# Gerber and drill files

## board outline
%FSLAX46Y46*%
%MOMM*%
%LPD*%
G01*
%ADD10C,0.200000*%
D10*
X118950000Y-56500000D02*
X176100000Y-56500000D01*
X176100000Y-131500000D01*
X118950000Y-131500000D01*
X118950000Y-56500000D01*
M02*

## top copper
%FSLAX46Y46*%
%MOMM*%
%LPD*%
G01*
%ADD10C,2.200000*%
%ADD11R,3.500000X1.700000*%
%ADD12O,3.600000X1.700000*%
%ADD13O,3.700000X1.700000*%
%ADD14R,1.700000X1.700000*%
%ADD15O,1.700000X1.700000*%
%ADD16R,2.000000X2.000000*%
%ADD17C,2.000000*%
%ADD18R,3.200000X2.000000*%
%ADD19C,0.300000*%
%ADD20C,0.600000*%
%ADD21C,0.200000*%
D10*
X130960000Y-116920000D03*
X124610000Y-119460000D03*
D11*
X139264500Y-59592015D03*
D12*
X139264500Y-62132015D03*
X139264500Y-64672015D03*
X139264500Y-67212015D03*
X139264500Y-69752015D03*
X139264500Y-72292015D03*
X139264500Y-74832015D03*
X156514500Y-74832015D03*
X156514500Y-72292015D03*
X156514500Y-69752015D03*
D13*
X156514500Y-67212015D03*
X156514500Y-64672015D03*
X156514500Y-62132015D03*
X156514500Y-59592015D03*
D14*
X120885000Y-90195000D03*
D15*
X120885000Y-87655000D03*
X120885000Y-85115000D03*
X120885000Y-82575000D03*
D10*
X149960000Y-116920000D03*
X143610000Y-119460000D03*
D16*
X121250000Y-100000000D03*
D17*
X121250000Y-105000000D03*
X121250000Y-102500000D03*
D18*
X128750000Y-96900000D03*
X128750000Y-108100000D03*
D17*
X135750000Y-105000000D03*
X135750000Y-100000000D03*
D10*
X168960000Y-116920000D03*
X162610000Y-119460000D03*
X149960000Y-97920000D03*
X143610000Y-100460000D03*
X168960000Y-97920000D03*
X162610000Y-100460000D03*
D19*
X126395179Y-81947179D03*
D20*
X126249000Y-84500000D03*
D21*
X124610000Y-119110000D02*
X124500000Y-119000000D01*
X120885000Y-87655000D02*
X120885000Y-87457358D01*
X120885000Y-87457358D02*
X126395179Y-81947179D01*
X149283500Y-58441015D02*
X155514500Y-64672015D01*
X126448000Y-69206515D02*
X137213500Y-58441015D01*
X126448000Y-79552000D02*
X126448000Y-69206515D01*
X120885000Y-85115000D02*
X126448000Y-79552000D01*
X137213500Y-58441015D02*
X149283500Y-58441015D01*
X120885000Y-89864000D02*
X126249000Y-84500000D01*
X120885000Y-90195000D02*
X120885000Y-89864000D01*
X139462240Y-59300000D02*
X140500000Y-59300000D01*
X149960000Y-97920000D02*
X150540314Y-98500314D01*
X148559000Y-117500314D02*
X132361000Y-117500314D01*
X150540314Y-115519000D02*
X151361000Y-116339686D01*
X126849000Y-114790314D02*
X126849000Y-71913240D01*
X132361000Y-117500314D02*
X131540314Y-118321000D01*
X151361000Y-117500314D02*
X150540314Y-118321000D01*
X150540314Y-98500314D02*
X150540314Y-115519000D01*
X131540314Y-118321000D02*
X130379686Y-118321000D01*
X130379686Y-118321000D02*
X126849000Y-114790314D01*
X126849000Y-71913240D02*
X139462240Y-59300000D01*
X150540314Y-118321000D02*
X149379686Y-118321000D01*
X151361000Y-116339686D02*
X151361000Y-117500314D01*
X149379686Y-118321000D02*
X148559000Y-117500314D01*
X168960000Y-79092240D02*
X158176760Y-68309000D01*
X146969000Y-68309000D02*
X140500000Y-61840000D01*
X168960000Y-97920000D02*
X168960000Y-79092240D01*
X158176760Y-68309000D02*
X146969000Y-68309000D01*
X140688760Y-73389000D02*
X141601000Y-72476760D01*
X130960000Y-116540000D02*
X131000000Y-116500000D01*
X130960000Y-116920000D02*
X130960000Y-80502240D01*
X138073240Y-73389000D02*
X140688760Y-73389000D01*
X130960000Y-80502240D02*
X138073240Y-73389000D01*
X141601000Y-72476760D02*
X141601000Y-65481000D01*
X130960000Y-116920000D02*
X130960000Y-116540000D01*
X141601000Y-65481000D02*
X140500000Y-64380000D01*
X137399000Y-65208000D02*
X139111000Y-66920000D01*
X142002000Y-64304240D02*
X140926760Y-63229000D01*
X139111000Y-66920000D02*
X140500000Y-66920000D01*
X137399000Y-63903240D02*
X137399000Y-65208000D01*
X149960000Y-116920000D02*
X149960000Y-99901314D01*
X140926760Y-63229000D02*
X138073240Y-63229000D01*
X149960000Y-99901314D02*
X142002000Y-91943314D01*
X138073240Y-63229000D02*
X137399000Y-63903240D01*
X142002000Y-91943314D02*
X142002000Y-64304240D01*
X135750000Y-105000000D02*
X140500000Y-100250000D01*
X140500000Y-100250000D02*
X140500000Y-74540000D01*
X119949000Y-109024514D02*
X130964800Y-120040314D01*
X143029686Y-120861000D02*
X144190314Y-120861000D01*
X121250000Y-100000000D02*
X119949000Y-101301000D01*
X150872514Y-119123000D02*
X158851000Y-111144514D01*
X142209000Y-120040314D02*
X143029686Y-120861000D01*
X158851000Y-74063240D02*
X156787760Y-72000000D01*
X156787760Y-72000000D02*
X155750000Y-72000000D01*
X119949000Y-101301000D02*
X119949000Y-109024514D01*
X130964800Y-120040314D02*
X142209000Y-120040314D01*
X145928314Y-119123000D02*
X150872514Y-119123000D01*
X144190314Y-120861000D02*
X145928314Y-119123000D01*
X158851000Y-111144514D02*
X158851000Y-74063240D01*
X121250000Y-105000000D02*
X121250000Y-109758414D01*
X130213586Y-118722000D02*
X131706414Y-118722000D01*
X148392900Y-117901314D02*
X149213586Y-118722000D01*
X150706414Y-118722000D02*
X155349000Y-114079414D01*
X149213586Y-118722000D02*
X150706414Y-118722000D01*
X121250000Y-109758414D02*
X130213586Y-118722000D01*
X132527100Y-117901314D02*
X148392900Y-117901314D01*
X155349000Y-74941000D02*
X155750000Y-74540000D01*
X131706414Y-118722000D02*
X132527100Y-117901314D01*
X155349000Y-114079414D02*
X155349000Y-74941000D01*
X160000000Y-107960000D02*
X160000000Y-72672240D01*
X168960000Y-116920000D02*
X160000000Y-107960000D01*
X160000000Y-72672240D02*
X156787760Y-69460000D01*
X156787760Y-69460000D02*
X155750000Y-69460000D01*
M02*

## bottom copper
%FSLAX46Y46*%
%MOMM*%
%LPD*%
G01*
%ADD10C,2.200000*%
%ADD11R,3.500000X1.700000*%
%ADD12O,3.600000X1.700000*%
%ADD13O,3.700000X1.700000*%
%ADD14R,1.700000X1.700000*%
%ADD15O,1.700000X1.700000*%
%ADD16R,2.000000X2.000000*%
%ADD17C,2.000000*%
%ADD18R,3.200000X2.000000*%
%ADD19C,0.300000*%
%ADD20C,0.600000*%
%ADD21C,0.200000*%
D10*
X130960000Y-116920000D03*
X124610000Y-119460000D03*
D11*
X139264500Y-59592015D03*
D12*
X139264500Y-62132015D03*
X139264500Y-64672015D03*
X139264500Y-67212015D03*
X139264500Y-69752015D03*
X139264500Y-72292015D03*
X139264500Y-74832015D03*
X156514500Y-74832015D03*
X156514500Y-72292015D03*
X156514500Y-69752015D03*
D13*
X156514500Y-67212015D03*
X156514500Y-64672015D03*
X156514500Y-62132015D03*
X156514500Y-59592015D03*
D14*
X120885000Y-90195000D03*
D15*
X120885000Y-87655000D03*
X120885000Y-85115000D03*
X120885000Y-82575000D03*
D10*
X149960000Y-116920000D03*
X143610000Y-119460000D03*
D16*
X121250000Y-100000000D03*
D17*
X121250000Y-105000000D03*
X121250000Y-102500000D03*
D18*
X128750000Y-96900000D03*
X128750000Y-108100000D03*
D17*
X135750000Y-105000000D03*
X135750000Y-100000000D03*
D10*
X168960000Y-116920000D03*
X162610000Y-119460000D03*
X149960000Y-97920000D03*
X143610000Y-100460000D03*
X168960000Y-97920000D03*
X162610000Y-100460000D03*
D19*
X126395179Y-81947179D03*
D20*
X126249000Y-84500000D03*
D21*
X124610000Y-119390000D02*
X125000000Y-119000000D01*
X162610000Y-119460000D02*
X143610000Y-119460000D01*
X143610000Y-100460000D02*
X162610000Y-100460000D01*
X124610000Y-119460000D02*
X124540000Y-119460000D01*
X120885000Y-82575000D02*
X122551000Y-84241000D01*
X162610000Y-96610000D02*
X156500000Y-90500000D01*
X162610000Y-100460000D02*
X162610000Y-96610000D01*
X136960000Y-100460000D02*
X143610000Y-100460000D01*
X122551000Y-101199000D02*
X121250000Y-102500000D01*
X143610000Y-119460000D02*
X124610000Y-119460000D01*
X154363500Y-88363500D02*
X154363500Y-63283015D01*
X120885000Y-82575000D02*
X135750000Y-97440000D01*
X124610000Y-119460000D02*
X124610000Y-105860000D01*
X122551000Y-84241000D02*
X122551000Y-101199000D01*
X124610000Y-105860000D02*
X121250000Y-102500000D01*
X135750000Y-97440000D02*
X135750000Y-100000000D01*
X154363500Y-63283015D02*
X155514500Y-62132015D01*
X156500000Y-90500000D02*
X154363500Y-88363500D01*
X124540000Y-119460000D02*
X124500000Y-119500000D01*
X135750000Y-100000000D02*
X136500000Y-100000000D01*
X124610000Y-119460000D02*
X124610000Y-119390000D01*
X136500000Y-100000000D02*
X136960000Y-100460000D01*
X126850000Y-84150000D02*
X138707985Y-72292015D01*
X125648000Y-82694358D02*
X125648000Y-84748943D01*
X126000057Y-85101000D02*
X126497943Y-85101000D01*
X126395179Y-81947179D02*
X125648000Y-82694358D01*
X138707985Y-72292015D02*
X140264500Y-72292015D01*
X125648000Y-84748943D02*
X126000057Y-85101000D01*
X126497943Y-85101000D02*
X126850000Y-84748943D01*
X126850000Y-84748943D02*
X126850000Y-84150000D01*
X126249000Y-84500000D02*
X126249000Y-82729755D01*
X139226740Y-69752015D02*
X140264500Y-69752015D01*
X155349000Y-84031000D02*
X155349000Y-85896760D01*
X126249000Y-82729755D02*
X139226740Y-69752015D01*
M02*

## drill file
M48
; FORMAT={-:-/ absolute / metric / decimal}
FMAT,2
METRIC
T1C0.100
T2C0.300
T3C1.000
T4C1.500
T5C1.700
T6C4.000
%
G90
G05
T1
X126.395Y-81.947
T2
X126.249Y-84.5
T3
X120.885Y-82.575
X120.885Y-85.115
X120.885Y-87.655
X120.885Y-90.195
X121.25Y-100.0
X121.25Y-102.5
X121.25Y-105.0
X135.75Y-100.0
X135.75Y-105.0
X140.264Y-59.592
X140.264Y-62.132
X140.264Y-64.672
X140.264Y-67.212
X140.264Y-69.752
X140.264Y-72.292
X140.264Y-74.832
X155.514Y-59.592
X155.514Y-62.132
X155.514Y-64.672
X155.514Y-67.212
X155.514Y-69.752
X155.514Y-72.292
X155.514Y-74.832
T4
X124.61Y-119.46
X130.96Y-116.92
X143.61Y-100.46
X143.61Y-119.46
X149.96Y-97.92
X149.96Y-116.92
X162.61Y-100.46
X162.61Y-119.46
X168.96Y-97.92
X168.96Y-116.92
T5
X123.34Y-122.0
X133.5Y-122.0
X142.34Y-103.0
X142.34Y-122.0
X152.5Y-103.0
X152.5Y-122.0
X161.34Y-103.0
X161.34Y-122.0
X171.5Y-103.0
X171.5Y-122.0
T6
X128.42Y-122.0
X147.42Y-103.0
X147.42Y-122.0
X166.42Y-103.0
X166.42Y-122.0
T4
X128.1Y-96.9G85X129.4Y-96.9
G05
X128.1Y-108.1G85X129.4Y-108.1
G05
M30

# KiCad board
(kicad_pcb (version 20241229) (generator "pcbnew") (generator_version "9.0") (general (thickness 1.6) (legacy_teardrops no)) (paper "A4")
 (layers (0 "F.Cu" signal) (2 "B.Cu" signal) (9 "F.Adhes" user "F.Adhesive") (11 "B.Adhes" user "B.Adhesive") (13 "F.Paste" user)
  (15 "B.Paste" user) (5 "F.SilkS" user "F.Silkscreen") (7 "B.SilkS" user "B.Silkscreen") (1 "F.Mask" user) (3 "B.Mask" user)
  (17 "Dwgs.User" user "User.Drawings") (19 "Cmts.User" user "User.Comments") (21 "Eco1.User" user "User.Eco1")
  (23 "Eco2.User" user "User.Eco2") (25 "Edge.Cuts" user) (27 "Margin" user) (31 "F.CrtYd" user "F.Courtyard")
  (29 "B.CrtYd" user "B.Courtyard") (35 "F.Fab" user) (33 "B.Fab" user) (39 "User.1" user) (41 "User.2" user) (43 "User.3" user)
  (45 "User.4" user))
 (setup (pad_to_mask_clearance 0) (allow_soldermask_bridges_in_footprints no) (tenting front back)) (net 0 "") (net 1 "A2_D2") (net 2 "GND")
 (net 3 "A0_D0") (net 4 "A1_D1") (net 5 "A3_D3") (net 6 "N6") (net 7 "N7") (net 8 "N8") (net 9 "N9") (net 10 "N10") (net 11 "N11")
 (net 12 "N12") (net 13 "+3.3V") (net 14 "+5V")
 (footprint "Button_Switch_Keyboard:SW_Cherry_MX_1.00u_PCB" (layer "F.Cu") (at 130.96 116.92)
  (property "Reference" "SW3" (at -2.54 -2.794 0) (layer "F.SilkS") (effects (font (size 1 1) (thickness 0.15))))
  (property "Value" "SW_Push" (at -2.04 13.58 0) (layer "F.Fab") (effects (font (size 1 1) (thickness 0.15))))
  (pad "" np_thru_hole circle (at -7.62 5.08) (size 1.7 1.7) (drill 1.7) (layers "*.Cu" "*.Mask"))
  (pad "" np_thru_hole circle (at -2.54 5.08) (size 4 4) (drill 4) (layers "*.Cu" "*.Mask"))
  (pad "" np_thru_hole circle (at 2.54 5.08) (size 1.7 1.7) (drill 1.7) (layers "*.Cu" "*.Mask"))
  (pad "1" thru_hole circle (at 0 0) (size 2.2 2.2) (drill 1.5) (layers "*.Cu" "*.Mask") (remove_unused_layers no) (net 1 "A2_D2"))
  (pad "2" thru_hole circle (at -6.35 2.54) (size 2.2 2.2) (drill 1.5) (layers "*.Cu" "*.Mask") (remove_unused_layers no) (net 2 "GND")))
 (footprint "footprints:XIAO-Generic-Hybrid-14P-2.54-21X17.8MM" (layer "F.Cu") (at 147.8895 67.212015)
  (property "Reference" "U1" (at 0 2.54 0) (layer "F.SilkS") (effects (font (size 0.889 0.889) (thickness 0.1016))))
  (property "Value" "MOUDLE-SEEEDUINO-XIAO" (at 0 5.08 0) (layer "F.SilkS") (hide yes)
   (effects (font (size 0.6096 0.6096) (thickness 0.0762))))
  (pad "1" thru_hole rect (at -7.625 -7.62) (size 3.5 1.7) (drill 1 (offset -1 0)) (layers "*.Cu" "*.Mask") (remove_unused_layers no)
   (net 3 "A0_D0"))
  (pad "2" thru_hole oval (at -7.625 -5.08) (size 3.6 1.7) (drill 1 (offset -1 0)) (layers "*.Cu" "*.Mask") (remove_unused_layers no)
   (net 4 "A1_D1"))
  (pad "3" thru_hole oval (at -7.625 -2.54) (size 3.6 1.7) (drill 1 (offset -1 0)) (layers "*.Cu" "*.Mask") (remove_unused_layers no)
   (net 1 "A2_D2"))
  (pad "4" thru_hole oval (at -7.625 0) (size 3.6 1.7) (drill 1 (offset -1 0)) (layers "*.Cu" "*.Mask") (remove_unused_layers no)
   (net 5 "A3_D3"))
  (pad "5" thru_hole oval (at -7.625 2.54) (size 3.6 1.7) (drill 1 (offset -1 0)) (layers "*.Cu" "*.Mask") (remove_unused_layers no)
   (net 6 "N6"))
  (pad "6" thru_hole oval (at -7.625 5.08 180) (size 3.6 1.7) (drill 1 (offset 1 0)) (layers "*.Cu" "*.Mask") (remove_unused_layers no)
   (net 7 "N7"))
  (pad "7" thru_hole oval (at -7.625 7.62) (size 3.6 1.7) (drill 1 (offset -1 0)) (layers "*.Cu" "*.Mask") (remove_unused_layers no)
   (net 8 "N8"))
  (pad "8" thru_hole oval (at 7.625 7.62) (size 3.6 1.7) (drill 1 (offset 1 0)) (layers "*.Cu" "*.Mask") (remove_unused_layers no)
   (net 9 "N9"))
  (pad "9" thru_hole oval (at 7.625 5.08) (size 3.6 1.7) (drill 1 (offset 1 0)) (layers "*.Cu" "*.Mask") (remove_unused_layers no)
   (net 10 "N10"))
  (pad "10" thru_hole oval (at 7.625 2.54) (size 3.6 1.7) (drill 1 (offset 1 0)) (layers "*.Cu" "*.Mask") (remove_unused_layers no)
   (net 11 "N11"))
  (pad "11" thru_hole oval (at 7.625 0) (size 3.7 1.7) (drill 1 (offset 1 0)) (layers "*.Cu" "*.Mask") (remove_unused_layers no)
   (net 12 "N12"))
  (pad "12" thru_hole oval (at 7.625 -2.54) (size 3.7 1.7) (drill 1 (offset 1 0)) (layers "*.Cu" "*.Mask") (remove_unused_layers no)
   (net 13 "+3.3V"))
  (pad "13" thru_hole oval (at 7.625 -5.08) (size 3.7 1.7) (drill 1 (offset 1 0)) (layers "*.Cu" "*.Mask") (remove_unused_layers no)
   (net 2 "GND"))
  (pad "14" thru_hole oval (at 7.625 -7.62) (size 3.7 1.7) (drill 1 (offset 1 0)) (layers "*.Cu" "*.Mask") (remove_unused_layers no)
   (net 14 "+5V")))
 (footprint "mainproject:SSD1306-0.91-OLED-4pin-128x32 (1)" (layer "F.Cu") (at 157.385 92.385 180)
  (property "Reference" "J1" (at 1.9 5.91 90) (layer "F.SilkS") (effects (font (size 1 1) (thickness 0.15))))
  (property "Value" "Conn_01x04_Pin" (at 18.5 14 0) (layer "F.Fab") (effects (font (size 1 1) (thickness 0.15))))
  (pad "1" thru_hole rect (at 36.5 2.19 180) (size 1.7 1.7) (drill 1) (layers "*.Cu" "*.Mask") (remove_unused_layers no) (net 6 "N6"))
  (pad "2" thru_hole oval (at 36.5 4.73 180) (size 1.7 1.7) (drill 1) (layers "*.Cu" "*.Mask") (remove_unused_layers no) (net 7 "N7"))
  (pad "3" thru_hole oval (at 36.5 7.27 180) (size 1.7 1.7) (drill 1) (layers "*.Cu" "*.Mask") (remove_unused_layers no) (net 13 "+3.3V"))
  (pad "4" thru_hole oval (at 36.5 9.81 180) (size 1.7 1.7) (drill 1) (layers "*.Cu" "*.Mask") (remove_unused_layers no) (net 2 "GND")))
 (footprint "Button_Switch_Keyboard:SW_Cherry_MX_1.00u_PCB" (layer "F.Cu") (at 149.96 116.92)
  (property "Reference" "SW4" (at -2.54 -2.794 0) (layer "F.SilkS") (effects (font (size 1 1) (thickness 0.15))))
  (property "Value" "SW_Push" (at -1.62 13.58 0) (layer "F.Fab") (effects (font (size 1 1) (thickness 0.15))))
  (pad "" np_thru_hole circle (at -7.62 5.08) (size 1.7 1.7) (drill 1.7) (layers "*.Cu" "*.Mask"))
  (pad "" np_thru_hole circle (at -2.54 5.08) (size 4 4) (drill 4) (layers "*.Cu" "*.Mask"))
  (pad "" np_thru_hole circle (at 2.54 5.08) (size 1.7 1.7) (drill 1.7) (layers "*.Cu" "*.Mask"))
  (pad "1" thru_hole circle (at 0 0) (size 2.2 2.2) (drill 1.5) (layers "*.Cu" "*.Mask") (remove_unused_layers no) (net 5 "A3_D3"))
  (pad "2" thru_hole circle (at -6.35 2.54) (size 2.2 2.2) (drill 1.5) (layers "*.Cu" "*.Mask") (remove_unused_layers no) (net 2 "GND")))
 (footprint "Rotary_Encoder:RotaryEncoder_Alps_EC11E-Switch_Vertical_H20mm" (layer "F.Cu") (at 121.25 100)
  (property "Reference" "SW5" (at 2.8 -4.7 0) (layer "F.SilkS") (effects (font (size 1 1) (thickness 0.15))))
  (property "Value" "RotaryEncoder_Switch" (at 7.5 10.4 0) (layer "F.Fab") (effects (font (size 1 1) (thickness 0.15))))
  (pad "A" thru_hole rect (at 0 0) (size 2 2) (drill 1) (layers "*.Cu" "*.Mask") (remove_unused_layers no) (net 10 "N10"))
  (pad "B" thru_hole circle (at 0 5) (size 2 2) (drill 1) (layers "*.Cu" "*.Mask") (remove_unused_layers no) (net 9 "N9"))
  (pad "C" thru_hole circle (at 0 2.5) (size 2 2) (drill 1) (layers "*.Cu" "*.Mask") (remove_unused_layers no) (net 2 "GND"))
  (pad "MP" thru_hole rect (at 7.5 -3.1) (size 3.2 2) (drill oval 2.8 1.5) (layers "*.Cu" "*.Mask") (remove_unused_layers no))
  (pad "MP" thru_hole rect (at 7.5 8.1) (size 3.2 2) (drill oval 2.8 1.5) (layers "*.Cu" "*.Mask") (remove_unused_layers no))
  (pad "S1" thru_hole circle (at 14.5 5) (size 2 2) (drill 1) (layers "*.Cu" "*.Mask") (remove_unused_layers no) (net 8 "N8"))
  (pad "S2" thru_hole circle (at 14.5 0) (size 2 2) (drill 1) (layers "*.Cu" "*.Mask") (remove_unused_layers no) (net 2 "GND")))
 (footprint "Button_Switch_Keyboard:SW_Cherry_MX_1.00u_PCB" (layer "F.Cu") (at 168.96 116.92)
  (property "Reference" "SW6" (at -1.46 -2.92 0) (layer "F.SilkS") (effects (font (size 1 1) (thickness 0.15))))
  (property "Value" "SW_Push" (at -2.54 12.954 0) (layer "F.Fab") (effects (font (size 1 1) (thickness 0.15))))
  (pad "" np_thru_hole circle (at -7.62 5.08) (size 1.7 1.7) (drill 1.7) (layers "*.Cu" "*.Mask"))
  (pad "" np_thru_hole circle (at -2.54 5.08) (size 4 4) (drill 4) (layers "*.Cu" "*.Mask"))
  (pad "" np_thru_hole circle (at 2.54 5.08) (size 1.7 1.7) (drill 1.7) (layers "*.Cu" "*.Mask"))
  (pad "1" thru_hole circle (at 0 0) (size 2.2 2.2) (drill 1.5) (layers "*.Cu" "*.Mask") (remove_unused_layers no) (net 11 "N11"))
  (pad "2" thru_hole circle (at -6.35 2.54) (size 2.2 2.2) (drill 1.5) (layers "*.Cu" "*.Mask") (remove_unused_layers no) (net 2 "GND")))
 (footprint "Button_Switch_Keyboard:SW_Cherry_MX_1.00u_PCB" (layer "F.Cu") (at 149.96 97.92)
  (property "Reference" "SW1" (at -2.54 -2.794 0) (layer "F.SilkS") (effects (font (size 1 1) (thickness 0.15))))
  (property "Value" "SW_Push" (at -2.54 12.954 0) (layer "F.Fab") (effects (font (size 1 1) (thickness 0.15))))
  (pad "" np_thru_hole circle (at -7.62 5.08) (size 1.7 1.7) (drill 1.7) (layers "*.Cu" "*.Mask"))
  (pad "" np_thru_hole circle (at -2.54 5.08) (size 4 4) (drill 4) (layers "*.Cu" "*.Mask"))
  (pad "" np_thru_hole circle (at 2.54 5.08) (size 1.7 1.7) (drill 1.7) (layers "*.Cu" "*.Mask"))
  (pad "1" thru_hole circle (at 0 0) (size 2.2 2.2) (drill 1.5) (layers "*.Cu" "*.Mask") (remove_unused_layers no) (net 3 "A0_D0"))
  (pad "2" thru_hole circle (at -6.35 2.54) (size 2.2 2.2) (drill 1.5) (layers "*.Cu" "*.Mask") (remove_unused_layers no) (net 2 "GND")))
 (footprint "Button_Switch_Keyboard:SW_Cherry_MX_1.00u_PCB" (layer "F.Cu") (at 168.96 97.92)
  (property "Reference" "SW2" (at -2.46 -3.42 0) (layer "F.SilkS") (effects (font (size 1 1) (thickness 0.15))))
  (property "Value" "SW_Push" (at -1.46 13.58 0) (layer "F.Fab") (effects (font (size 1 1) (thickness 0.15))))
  (pad "" np_thru_hole circle (at -7.62 5.08) (size 1.7 1.7) (drill 1.7) (layers "*.Cu" "*.Mask"))
  (pad "" np_thru_hole circle (at -2.54 5.08) (size 4 4) (drill 4) (layers "*.Cu" "*.Mask"))
  (pad "" np_thru_hole circle (at 2.54 5.08) (size 1.7 1.7) (drill 1.7) (layers "*.Cu" "*.Mask"))
  (pad "1" thru_hole circle (at 0 0) (size 2.2 2.2) (drill 1.5) (layers "*.Cu" "*.Mask") (remove_unused_layers no) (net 4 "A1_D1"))
  (pad "2" thru_hole circle (at -6.35 2.54) (size 2.2 2.2) (drill 1.5) (layers "*.Cu" "*.Mask") (remove_unused_layers no) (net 2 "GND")))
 (gr_rect (start 118.95 56.5) (end 176.1 131.5) (stroke (width 0.2) (type solid)) (fill no) (layer "Edge.Cuts"))
 (segment (start 124.61 119.11) (end 124.5 119) (width 0.2) (layer "F.Cu") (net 2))
 (segment (start 124.61 119.39) (end 125 119) (width 0.2) (layer "B.Cu") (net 2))
 (segment (start 162.61 119.46) (end 143.61 119.46) (width 0.2) (layer "B.Cu") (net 2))
 (segment (start 143.61 100.46) (end 162.61 100.46) (width 0.2) (layer "B.Cu") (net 2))
 (segment (start 124.61 119.46) (end 124.54 119.46) (width 0.2) (layer "B.Cu") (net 2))
 (segment (start 120.885 82.575) (end 122.551 84.241) (width 0.2) (layer "B.Cu") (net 2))
 (segment (start 162.61 96.61) (end 156.5 90.5) (width 0.2) (layer "B.Cu") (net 2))
 (segment (start 162.61 100.46) (end 162.61 96.61) (width 0.2) (layer "B.Cu") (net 2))
 (segment (start 136.96 100.46) (end 143.61 100.46) (width 0.2) (layer "B.Cu") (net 2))
 (segment (start 122.551 101.199) (end 121.25 102.5) (width 0.2) (layer "B.Cu") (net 2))
 (segment (start 143.61 119.46) (end 124.61 119.46) (width 0.2) (layer "B.Cu") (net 2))
 (segment (start 154.3635 88.3635) (end 154.3635 63.283015) (width 0.2) (layer "B.Cu") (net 2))
 (segment (start 120.885 82.575) (end 135.75 97.44) (width 0.2) (layer "B.Cu") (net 2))
 (segment (start 124.61 119.46) (end 124.61 105.86) (width 0.2) (layer "B.Cu") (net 2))
 (segment (start 122.551 84.241) (end 122.551 101.199) (width 0.2) (layer "B.Cu") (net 2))
 (segment (start 124.61 105.86) (end 121.25 102.5) (width 0.2) (layer "B.Cu") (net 2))
 (segment (start 135.75 97.44) (end 135.75 100) (width 0.2) (layer "B.Cu") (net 2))
 (segment (start 154.3635 63.283015) (end 155.5145 62.132015) (width 0.2) (layer "B.Cu") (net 2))
 (segment (start 156.5 90.5) (end 154.3635 88.3635) (width 0.2) (layer "B.Cu") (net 2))
 (segment (start 124.54 119.46) (end 124.5 119.5) (width 0.2) (layer "B.Cu") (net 2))
 (segment (start 135.75 100) (end 136.5 100) (width 0.2) (layer "B.Cu") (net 2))
 (segment (start 124.61 119.46) (end 124.61 119.39) (width 0.2) (layer "B.Cu") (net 2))
 (segment (start 136.5 100) (end 136.96 100.46) (width 0.2) (layer "B.Cu") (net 2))
 (segment (start 120.885 87.655) (end 120.885 87.457358) (width 0.2) (layer "F.Cu") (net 7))
 (segment (start 120.885 87.457358) (end 126.395179 81.947179) (width 0.2) (layer "F.Cu") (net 7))
 (via micro (at 126.395179 81.947179) (size 0.3) (drill 0.1) (layers "F.Cu" "B.Cu") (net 7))
 (segment (start 126.85 84.15) (end 138.707985 72.292015) (width 0.2) (layer "B.Cu") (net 7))
 (segment (start 125.648 82.694358) (end 125.648 84.748943) (width 0.2) (layer "B.Cu") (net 7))
 (segment (start 126.000057 85.101) (end 126.497943 85.101) (width 0.2) (layer "B.Cu") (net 7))
 (segment (start 126.395179 81.947179) (end 125.648 82.694358) (width 0.2) (layer "B.Cu") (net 7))
 (segment (start 138.707985 72.292015) (end 140.2645 72.292015) (width 0.2) (layer "B.Cu") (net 7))
 (segment (start 125.648 84.748943) (end 126.000057 85.101) (width 0.2) (layer "B.Cu") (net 7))
 (segment (start 126.497943 85.101) (end 126.85 84.748943) (width 0.2) (layer "B.Cu") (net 7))
 (segment (start 126.85 84.748943) (end 126.85 84.15) (width 0.2) (layer "B.Cu") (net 7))
 (segment (start 149.2835 58.441015) (end 155.5145 64.672015) (width 0.2) (layer "F.Cu") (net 13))
 (segment (start 126.448 69.206515) (end 137.2135 58.441015) (width 0.2) (layer "F.Cu") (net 13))
 (segment (start 126.448 79.552) (end 126.448 69.206515) (width 0.2) (layer "F.Cu") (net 13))
 (segment (start 120.885 85.115) (end 126.448 79.552) (width 0.2) (layer "F.Cu") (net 13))
 (segment (start 137.2135 58.441015) (end 149.2835 58.441015) (width 0.2) (layer "F.Cu") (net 13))
 (segment (start 120.885 89.864) (end 126.249 84.5) (width 0.2) (layer "F.Cu") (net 6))
 (segment (start 120.885 90.195) (end 120.885 89.864) (width 0.2) (layer "F.Cu") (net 6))
 (via blind (at 126.249 84.5) (size 0.6) (drill 0.3) (layers "F.Cu" "B.Cu") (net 6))
 (segment (start 126.249 84.5) (end 126.249 82.729755) (width 0.2) (layer "B.Cu") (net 6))
 (segment (start 139.22674 69.752015) (end 140.2645 69.752015) (width 0.2) (layer "B.Cu") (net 6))
 (segment (start 155.349 84.031) (end 155.349 85.89676) (width 0.2) (layer "B.Cu") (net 6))
 (segment (start 126.249 82.729755) (end 139.22674 69.752015) (width 0.2) (layer "B.Cu") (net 6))
 (segment (start 139.46224 59.3) (end 140.5 59.3) (width 0.2) (layer "F.Cu") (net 3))
 (segment (start 149.96 97.92) (end 150.540314 98.500314) (width 0.2) (layer "F.Cu") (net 3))
 (segment (start 148.559 117.500314) (end 132.361 117.500314) (width 0.2) (layer "F.Cu") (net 3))
 (segment (start 150.540314 115.519) (end 151.361 116.339686) (width 0.2) (layer "F.Cu") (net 3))
 (segment (start 126.849 114.790314) (end 126.849 71.91324) (width 0.2) (layer "F.Cu") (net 3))
 (segment (start 132.361 117.500314) (end 131.540314 118.321) (width 0.2) (layer "F.Cu") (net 3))
 (segment (start 151.361 117.500314) (end 150.540314 118.321) (width 0.2) (layer "F.Cu") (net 3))
 (segment (start 150.540314 98.500314) (end 150.540314 115.519) (width 0.2) (layer "F.Cu") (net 3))
 (segment (start 131.540314 118.321) (end 130.379686 118.321) (width 0.2) (layer "F.Cu") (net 3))
 (segment (start 130.379686 118.321) (end 126.849 114.790314) (width 0.2) (layer "F.Cu") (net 3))
 (segment (start 126.849 71.91324) (end 139.46224 59.3) (width 0.2) (layer "F.Cu") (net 3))
 (segment (start 150.540314 118.321) (end 149.379686 118.321) (width 0.2) (layer "F.Cu") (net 3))
 (segment (start 151.361 116.339686) (end 151.361 117.500314) (width 0.2) (layer "F.Cu") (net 3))
 (segment (start 149.379686 118.321) (end 148.559 117.500314) (width 0.2) (layer "F.Cu") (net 3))
 (segment (start 168.96 79.09224) (end 158.17676 68.309) (width 0.2) (layer "F.Cu") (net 4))
 (segment (start 146.969 68.309) (end 140.5 61.84) (width 0.2) (layer "F.Cu") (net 4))
 (segment (start 168.96 97.92) (end 168.96 79.09224) (width 0.2) (layer "F.Cu") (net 4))
 (segment (start 158.17676 68.309) (end 146.969 68.309) (width 0.2) (layer "F.Cu") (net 4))
 (segment (start 140.68876 73.389) (end 141.601 72.47676) (width 0.2) (layer "F.Cu") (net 1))
 (segment (start 130.96 116.54) (end 131 116.5) (width 0.2) (layer "F.Cu") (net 1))
 (segment (start 130.96 116.92) (end 130.96 80.50224) (width 0.2) (layer "F.Cu") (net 1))
 (segment (start 138.07324 73.389) (end 140.68876 73.389) (width 0.2) (layer "F.Cu") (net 1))
 (segment (start 130.96 80.50224) (end 138.07324 73.389) (width 0.2) (layer "F.Cu") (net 1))
 (segment (start 141.601 72.47676) (end 141.601 65.481) (width 0.2) (layer "F.Cu") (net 1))
 (segment (start 130.96 116.92) (end 130.96 116.54) (width 0.2) (layer "F.Cu") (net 1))
 (segment (start 141.601 65.481) (end 140.5 64.38) (width 0.2) (layer "F.Cu") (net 1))
 (segment (start 137.399 65.208) (end 139.111 66.92) (width 0.2) (layer "F.Cu") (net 5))
 (segment (start 142.002 64.30424) (end 140.92676 63.229) (width 0.2) (layer "F.Cu") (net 5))
 (segment (start 139.111 66.92) (end 140.5 66.92) (width 0.2) (layer "F.Cu") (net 5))
 (segment (start 137.399 63.90324) (end 137.399 65.208) (width 0.2) (layer "F.Cu") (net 5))
 (segment (start 149.96 116.92) (end 149.96 99.901314) (width 0.2) (layer "F.Cu") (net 5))
 (segment (start 140.92676 63.229) (end 138.07324 63.229) (width 0.2) (layer "F.Cu") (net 5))
 (segment (start 149.96 99.901314) (end 142.002 91.943314) (width 0.2) (layer "F.Cu") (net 5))
 (segment (start 138.07324 63.229) (end 137.399 63.90324) (width 0.2) (layer "F.Cu") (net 5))
 (segment (start 142.002 91.943314) (end 142.002 64.30424) (width 0.2) (layer "F.Cu") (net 5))
 (segment (start 135.75 105) (end 140.5 100.25) (width 0.2) (layer "F.Cu") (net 8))
 (segment (start 140.5 100.25) (end 140.5 74.54) (width 0.2) (layer "F.Cu") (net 8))
 (segment (start 119.949 109.024514) (end 130.9648 120.040314) (width 0.2) (layer "F.Cu") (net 10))
 (segment (start 143.029686 120.861) (end 144.190314 120.861) (width 0.2) (layer "F.Cu") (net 10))
 (segment (start 121.25 100) (end 119.949 101.301) (width 0.2) (layer "F.Cu") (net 10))
 (segment (start 150.872514 119.123) (end 158.851 111.144514) (width 0.2) (layer "F.Cu") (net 10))
 (segment (start 142.209 120.040314) (end 143.029686 120.861) (width 0.2) (layer "F.Cu") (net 10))
 (segment (start 158.851 74.06324) (end 156.78776 72) (width 0.2) (layer "F.Cu") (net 10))
 (segment (start 156.78776 72) (end 155.75 72) (width 0.2) (layer "F.Cu") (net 10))
 (segment (start 119.949 101.301) (end 119.949 109.024514) (width 0.2) (layer "F.Cu") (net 10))
 (segment (start 130.9648 120.040314) (end 142.209 120.040314) (width 0.2) (layer "F.Cu") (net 10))
 (segment (start 145.928314 119.123) (end 150.872514 119.123) (width 0.2) (layer "F.Cu") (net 10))
 (segment (start 144.190314 120.861) (end 145.928314 119.123) (width 0.2) (layer "F.Cu") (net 10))
 (segment (start 158.851 111.144514) (end 158.851 74.06324) (width 0.2) (layer "F.Cu") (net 10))
 (segment (start 121.25 105) (end 121.25 109.758414) (width 0.2) (layer "F.Cu") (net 9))
 (segment (start 130.213586 118.722) (end 131.706414 118.722) (width 0.2) (layer "F.Cu") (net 9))
 (segment (start 148.3929 117.901314) (end 149.213586 118.722) (width 0.2) (layer "F.Cu") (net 9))
 (segment (start 150.706414 118.722) (end 155.349 114.079414) (width 0.2) (layer "F.Cu") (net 9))
 (segment (start 149.213586 118.722) (end 150.706414 118.722) (width 0.2) (layer "F.Cu") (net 9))
 (segment (start 121.25 109.758414) (end 130.213586 118.722) (width 0.2) (layer "F.Cu") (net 9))
 (segment (start 132.5271 117.901314) (end 148.3929 117.901314) (width 0.2) (layer "F.Cu") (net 9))
 (segment (start 155.349 74.941) (end 155.75 74.54) (width 0.2) (layer "F.Cu") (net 9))
 (segment (start 131.706414 118.722) (end 132.5271 117.901314) (width 0.2) (layer "F.Cu") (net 9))
 (segment (start 155.349 114.079414) (end 155.349 74.941) (width 0.2) (layer "F.Cu") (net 9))
 (segment (start 160 107.96) (end 160 72.67224) (width 0.2) (layer "F.Cu") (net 11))
 (segment (start 168.96 116.92) (end 160 107.96) (width 0.2) (layer "F.Cu") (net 11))
 (segment (start 160 72.67224) (end 156.78776 69.46) (width 0.2) (layer "F.Cu") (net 11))
 (segment (start 156.78776 69.46) (end 155.75 69.46) (width 0.2) (layer "F.Cu") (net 11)))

